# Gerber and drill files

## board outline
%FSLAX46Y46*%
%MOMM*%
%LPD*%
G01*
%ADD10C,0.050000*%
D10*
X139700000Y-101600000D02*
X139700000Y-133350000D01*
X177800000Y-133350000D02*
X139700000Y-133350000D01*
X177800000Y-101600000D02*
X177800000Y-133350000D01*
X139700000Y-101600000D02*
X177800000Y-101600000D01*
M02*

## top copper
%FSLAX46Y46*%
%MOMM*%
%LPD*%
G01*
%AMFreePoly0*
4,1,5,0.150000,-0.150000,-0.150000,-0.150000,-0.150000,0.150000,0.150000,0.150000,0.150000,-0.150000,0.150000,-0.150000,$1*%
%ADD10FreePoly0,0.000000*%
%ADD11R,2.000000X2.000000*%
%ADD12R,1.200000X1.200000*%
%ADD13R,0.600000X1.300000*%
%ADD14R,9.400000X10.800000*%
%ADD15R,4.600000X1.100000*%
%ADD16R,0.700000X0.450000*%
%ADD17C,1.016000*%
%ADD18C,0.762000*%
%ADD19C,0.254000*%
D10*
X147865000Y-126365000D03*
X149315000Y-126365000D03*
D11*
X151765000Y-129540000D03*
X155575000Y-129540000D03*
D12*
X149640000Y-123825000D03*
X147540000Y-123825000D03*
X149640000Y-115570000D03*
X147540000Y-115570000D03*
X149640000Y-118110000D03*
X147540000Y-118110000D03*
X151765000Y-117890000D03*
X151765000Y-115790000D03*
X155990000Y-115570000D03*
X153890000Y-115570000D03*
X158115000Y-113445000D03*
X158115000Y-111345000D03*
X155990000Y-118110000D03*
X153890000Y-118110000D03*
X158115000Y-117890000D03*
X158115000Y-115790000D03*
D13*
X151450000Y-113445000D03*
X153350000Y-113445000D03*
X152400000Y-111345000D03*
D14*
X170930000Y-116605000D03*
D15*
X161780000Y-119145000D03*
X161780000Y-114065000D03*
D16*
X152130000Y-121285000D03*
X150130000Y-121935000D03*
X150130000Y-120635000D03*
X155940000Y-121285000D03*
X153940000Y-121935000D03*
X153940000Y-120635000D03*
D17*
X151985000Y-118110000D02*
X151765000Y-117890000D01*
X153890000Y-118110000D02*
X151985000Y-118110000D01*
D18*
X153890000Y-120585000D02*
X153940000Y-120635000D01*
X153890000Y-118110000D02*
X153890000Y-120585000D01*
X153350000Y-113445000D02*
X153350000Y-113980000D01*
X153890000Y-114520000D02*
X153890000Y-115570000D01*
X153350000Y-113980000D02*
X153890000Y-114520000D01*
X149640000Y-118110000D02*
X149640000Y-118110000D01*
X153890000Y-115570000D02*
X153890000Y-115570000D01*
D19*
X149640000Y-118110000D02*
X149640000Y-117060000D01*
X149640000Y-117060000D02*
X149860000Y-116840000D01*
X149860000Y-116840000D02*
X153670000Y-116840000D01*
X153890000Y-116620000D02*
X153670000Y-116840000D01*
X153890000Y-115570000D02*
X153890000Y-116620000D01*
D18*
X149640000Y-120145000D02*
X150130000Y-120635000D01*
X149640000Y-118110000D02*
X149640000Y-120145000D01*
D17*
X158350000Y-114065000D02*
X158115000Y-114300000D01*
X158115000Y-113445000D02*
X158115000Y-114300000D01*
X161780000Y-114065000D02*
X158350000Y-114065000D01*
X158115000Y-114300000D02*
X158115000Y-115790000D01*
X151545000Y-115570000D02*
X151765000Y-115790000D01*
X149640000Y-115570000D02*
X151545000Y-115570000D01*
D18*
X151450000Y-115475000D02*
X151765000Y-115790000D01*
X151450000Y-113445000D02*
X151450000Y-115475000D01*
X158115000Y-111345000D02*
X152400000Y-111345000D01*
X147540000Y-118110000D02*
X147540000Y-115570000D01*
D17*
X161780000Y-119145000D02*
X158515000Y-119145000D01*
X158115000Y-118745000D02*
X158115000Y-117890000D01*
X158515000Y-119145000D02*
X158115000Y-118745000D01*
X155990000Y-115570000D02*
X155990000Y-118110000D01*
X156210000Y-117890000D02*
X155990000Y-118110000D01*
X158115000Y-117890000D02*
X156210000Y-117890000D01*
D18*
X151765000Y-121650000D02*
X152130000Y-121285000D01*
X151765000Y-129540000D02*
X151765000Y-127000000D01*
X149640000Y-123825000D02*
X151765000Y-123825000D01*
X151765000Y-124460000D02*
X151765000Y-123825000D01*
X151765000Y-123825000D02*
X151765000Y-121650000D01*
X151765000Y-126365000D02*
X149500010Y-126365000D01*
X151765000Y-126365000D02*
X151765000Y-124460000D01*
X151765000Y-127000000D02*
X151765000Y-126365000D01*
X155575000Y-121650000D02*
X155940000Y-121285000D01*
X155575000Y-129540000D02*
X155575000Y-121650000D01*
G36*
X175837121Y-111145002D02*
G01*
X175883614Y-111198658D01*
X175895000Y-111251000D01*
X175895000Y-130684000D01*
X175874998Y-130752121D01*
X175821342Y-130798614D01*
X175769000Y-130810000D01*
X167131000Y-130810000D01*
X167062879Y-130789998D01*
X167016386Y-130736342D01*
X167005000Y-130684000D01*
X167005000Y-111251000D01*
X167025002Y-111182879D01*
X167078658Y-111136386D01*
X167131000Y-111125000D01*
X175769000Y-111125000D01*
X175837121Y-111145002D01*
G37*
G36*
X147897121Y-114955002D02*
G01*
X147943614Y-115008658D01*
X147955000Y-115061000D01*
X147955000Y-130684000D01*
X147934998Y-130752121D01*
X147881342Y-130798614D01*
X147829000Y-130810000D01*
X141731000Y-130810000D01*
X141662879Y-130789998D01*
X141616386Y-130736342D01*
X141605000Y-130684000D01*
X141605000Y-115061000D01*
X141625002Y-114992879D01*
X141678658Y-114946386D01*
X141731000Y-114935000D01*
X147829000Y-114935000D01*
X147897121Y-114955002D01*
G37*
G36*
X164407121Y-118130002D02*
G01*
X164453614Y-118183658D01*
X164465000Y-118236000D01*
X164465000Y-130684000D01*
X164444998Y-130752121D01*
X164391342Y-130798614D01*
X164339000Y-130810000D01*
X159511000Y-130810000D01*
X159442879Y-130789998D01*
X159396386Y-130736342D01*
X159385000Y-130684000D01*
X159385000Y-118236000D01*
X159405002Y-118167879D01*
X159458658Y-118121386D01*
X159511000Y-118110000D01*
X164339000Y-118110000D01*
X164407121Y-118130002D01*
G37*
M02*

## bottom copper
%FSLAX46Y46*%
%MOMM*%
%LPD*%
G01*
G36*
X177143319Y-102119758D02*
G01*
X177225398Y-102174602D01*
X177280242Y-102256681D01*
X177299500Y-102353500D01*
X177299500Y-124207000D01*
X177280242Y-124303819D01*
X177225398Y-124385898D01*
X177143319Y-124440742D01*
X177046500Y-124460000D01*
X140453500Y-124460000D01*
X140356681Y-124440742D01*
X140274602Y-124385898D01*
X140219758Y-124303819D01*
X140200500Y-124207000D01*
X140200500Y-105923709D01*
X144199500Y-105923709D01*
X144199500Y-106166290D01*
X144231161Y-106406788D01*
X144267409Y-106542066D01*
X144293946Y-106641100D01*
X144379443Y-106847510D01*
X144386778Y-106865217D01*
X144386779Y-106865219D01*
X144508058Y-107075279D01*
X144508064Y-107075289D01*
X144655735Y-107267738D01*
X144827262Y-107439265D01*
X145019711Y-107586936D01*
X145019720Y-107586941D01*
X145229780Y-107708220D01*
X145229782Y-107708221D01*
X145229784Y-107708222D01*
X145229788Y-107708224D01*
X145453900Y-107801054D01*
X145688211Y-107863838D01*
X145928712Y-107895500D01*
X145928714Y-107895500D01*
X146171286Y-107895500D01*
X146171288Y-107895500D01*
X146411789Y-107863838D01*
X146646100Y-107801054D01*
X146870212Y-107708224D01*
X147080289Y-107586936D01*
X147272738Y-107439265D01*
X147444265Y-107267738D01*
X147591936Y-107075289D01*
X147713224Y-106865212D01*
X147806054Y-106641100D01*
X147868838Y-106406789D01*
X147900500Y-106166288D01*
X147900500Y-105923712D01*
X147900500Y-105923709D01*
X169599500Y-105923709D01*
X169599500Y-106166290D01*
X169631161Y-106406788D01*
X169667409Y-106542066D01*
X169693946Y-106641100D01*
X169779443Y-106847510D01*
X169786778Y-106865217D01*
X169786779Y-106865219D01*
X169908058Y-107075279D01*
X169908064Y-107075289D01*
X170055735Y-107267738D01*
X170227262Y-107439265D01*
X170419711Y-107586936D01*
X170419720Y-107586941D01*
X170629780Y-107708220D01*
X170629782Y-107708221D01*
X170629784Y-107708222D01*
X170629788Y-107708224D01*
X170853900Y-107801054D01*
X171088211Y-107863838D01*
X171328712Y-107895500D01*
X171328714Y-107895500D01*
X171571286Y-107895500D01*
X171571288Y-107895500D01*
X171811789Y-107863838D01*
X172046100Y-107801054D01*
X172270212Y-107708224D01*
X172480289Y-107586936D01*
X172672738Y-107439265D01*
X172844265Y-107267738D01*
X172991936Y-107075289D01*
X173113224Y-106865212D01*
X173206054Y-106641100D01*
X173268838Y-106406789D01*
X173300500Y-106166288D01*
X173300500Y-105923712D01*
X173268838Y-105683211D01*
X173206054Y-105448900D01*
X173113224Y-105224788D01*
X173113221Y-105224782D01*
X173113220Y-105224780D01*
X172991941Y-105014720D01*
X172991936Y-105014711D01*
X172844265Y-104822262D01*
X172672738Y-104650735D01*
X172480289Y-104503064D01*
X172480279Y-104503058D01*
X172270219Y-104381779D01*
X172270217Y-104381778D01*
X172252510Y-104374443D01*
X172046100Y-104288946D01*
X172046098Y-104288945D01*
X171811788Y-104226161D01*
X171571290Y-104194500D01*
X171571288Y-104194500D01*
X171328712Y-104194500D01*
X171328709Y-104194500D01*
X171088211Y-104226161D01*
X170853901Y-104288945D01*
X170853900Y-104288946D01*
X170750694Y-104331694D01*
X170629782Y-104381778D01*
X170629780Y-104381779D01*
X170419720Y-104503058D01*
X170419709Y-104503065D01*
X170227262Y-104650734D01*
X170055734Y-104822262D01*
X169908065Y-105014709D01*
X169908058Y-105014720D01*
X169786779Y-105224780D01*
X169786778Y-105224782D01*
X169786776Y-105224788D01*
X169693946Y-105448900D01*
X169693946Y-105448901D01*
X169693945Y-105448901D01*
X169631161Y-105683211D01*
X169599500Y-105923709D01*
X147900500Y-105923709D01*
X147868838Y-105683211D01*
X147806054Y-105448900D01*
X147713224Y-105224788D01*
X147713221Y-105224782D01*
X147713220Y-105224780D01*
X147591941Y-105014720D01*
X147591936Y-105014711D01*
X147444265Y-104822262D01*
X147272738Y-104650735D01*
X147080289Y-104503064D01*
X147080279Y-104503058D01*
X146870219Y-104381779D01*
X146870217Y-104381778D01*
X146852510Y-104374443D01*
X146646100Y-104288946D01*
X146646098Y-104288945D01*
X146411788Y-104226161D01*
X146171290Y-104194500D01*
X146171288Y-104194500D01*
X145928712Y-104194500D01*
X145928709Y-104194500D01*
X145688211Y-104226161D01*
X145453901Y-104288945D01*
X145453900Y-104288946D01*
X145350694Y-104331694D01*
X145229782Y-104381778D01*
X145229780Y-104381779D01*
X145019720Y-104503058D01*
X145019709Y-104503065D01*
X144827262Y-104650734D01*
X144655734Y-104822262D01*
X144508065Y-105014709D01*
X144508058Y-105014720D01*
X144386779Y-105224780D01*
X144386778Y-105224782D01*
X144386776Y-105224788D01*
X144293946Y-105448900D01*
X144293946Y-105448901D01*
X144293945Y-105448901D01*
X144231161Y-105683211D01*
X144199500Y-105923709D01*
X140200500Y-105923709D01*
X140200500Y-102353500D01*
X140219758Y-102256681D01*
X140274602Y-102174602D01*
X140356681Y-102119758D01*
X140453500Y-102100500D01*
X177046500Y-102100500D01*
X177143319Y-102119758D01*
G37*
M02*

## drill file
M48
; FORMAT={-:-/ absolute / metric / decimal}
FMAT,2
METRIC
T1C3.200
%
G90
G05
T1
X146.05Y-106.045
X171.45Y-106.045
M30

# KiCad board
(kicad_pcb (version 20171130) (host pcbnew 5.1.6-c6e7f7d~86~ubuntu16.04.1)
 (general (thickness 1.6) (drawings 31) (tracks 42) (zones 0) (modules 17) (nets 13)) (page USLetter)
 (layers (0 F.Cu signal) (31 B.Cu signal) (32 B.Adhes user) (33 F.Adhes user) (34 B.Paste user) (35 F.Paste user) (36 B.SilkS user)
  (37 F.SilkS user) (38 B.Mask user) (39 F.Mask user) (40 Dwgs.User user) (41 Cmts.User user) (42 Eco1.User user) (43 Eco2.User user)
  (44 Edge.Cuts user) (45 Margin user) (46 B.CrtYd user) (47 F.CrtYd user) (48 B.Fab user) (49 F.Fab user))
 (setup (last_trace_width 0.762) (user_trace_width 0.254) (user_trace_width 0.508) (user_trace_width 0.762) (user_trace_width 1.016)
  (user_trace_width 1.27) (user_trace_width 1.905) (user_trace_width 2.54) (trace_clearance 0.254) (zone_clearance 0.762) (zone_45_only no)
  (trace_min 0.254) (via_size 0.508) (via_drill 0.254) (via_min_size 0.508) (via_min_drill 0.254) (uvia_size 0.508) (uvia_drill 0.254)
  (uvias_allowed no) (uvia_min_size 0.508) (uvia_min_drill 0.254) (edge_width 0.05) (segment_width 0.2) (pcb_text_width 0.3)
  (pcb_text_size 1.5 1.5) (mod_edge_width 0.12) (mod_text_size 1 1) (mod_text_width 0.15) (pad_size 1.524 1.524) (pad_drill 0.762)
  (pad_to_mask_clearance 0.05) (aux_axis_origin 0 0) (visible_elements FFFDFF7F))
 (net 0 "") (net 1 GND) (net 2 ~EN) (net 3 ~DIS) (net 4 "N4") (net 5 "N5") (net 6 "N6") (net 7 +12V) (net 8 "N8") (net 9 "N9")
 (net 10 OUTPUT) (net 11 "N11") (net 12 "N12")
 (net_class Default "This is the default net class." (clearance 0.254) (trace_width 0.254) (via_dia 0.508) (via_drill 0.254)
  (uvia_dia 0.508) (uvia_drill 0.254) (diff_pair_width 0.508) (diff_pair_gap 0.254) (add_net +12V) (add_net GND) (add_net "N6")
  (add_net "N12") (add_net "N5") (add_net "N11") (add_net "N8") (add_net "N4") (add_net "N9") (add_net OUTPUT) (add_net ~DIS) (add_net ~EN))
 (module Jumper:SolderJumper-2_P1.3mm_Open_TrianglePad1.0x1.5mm (layer F.Cu) (at 148.59 126.365)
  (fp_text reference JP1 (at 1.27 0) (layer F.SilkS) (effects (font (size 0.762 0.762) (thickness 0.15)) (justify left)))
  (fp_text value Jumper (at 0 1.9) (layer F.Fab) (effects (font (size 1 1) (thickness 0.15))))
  (pad 1 smd custom (at -0.725 0) (size 0.3 0.3) (layers F.Cu F.Mask) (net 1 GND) (zone_connect 2)
   (options (clearance outline) (anchor rect)) (primitives))
  (pad 2 smd custom (at 0.725 0) (size 0.3 0.3) (layers F.Cu F.Mask) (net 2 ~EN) (zone_connect 2)
   (options (clearance outline) (anchor rect)) (primitives)))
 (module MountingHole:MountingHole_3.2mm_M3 (layer F.Cu) (at 171.45 106.045)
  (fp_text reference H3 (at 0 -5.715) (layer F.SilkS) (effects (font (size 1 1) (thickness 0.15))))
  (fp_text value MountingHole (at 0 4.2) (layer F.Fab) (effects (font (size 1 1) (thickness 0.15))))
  (pad 1 np_thru_hole circle (at 0 0) (size 3.2 3.2) (drill 3.2) (layers *.Cu *.Mask)))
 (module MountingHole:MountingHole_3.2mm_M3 (layer F.Cu) (at 146.05 106.045)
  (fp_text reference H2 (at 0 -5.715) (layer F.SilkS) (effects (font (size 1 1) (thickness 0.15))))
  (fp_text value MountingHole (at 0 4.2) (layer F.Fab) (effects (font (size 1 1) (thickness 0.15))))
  (pad 1 np_thru_hole circle (at 0 0) (size 3.2 3.2) (drill 3.2) (layers *.Cu *.Mask)))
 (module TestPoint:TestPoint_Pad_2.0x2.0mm (layer F.Cu) (at 151.765 129.54 180)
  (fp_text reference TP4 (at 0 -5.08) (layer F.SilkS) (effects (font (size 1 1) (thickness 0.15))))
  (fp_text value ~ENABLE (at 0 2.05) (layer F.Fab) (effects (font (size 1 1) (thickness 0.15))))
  (pad 1 smd rect (at 0 0 180) (size 2 2) (layers F.Cu F.Mask) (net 2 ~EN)))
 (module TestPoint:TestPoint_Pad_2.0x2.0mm (layer F.Cu) (at 155.575 129.54 180)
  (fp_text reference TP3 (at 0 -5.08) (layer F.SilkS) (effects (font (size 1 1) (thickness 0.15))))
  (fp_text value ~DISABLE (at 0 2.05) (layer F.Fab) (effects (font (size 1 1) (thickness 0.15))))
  (pad 1 smd rect (at 0 0 180) (size 2 2) (layers F.Cu F.Mask) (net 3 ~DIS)))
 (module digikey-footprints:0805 (layer F.Cu) (at 148.59 123.825 180)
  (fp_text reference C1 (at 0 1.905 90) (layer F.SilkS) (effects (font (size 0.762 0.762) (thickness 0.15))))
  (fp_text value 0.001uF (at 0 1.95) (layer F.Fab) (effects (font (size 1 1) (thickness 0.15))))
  (pad 1 smd rect (at -1.05 0 180) (size 1.2 1.2) (layers F.Cu F.Paste F.Mask) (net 2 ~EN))
  (pad 2 smd rect (at 1.05 0 180) (size 1.2 1.2) (layers F.Cu F.Paste F.Mask) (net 1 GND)))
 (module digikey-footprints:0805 (layer F.Cu) (at 148.59 115.57 180)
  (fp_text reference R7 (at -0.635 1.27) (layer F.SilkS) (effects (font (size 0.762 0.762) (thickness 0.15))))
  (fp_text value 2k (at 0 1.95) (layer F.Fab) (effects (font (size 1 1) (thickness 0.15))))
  (pad 1 smd rect (at -1.05 0 180) (size 1.2 1.2) (layers F.Cu F.Paste F.Mask) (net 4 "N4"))
  (pad 2 smd rect (at 1.05 0 180) (size 1.2 1.2) (layers F.Cu F.Paste F.Mask) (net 1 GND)))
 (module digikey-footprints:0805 (layer F.Cu) (at 148.59 118.11 180)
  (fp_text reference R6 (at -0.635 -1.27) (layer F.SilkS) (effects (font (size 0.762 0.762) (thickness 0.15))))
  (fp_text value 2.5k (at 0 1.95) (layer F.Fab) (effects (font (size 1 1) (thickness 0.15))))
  (pad 1 smd rect (at -1.05 0 180) (size 1.2 1.2) (layers F.Cu F.Paste F.Mask) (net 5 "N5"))
  (pad 2 smd rect (at 1.05 0 180) (size 1.2 1.2) (layers F.Cu F.Paste F.Mask) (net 1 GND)))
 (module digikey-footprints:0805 (layer F.Cu) (at 151.765 116.84 90)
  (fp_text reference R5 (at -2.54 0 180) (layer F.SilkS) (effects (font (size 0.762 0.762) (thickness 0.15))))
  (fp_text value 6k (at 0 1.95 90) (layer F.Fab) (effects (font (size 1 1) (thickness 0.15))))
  (pad 1 smd rect (at -1.05 0 90) (size 1.2 1.2) (layers F.Cu F.Paste F.Mask) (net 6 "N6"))
  (pad 2 smd rect (at 1.05 0 90) (size 1.2 1.2) (layers F.Cu F.Paste F.Mask) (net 4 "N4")))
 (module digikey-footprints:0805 (layer F.Cu) (at 154.94 115.57 180)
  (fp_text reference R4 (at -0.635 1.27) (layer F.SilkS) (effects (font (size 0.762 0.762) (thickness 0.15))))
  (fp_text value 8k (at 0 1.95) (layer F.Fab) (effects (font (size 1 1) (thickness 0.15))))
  (pad 1 smd rect (at -1.05 0 180) (size 1.2 1.2) (layers F.Cu F.Paste F.Mask) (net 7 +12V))
  (pad 2 smd rect (at 1.05 0 180) (size 1.2 1.2) (layers F.Cu F.Paste F.Mask) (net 5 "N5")))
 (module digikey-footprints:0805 (layer F.Cu) (at 158.115 112.395 90)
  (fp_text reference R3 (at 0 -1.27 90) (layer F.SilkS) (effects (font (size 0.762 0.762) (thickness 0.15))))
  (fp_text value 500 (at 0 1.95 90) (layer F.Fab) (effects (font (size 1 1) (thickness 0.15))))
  (pad 1 smd rect (at -1.05 0 90) (size 1.2 1.2) (layers F.Cu F.Paste F.Mask) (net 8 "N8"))
  (pad 2 smd rect (at 1.05 0 90) (size 1.2 1.2) (layers F.Cu F.Paste F.Mask) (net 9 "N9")))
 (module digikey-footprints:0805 (layer F.Cu) (at 154.94 118.11 180)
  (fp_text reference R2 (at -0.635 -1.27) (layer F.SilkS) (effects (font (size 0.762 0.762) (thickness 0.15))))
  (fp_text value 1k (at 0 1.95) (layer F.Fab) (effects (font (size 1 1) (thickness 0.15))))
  (pad 1 smd rect (at -1.05 0 180) (size 1.2 1.2) (layers F.Cu F.Paste F.Mask) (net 7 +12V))
  (pad 2 smd rect (at 1.05 0 180) (size 1.2 1.2) (layers F.Cu F.Paste F.Mask) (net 6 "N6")))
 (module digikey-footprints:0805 (layer F.Cu) (at 158.115 116.84 90)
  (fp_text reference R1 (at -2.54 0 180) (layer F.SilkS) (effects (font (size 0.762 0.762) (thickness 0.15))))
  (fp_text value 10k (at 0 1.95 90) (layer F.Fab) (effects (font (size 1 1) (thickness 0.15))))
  (pad 1 smd rect (at -1.05 0 90) (size 1.2 1.2) (layers F.Cu F.Paste F.Mask) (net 7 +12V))
  (pad 2 smd rect (at 1.05 0 90) (size 1.2 1.2) (layers F.Cu F.Paste F.Mask) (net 8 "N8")))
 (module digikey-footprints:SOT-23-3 (layer F.Cu) (at 152.4 112.395 90)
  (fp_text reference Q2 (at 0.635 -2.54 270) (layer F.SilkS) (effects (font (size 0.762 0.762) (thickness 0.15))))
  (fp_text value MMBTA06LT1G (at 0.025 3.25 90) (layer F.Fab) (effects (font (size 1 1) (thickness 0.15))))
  (pad 1 smd rect (at -1.05 -0.95 90) (size 1.3 0.6) (layers F.Cu F.Paste F.Mask) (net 4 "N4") (solder_mask_margin 0.07))
  (pad 2 smd rect (at -1.05 0.95 90) (size 1.3 0.6) (layers F.Cu F.Paste F.Mask) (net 5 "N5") (solder_mask_margin 0.07))
  (pad 3 smd rect (at 1.05 0 90) (size 1.3 0.6) (layers F.Cu F.Paste F.Mask) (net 9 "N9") (solder_mask_margin 0.07)))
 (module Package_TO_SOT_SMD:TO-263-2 (layer F.Cu) (at 167.555 116.605)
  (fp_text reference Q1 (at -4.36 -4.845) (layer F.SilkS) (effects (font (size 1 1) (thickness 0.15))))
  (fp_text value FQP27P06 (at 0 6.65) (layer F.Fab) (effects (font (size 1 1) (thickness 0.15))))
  (pad "" smd rect (at 0.95 2.775) (size 4.55 5.25) (layers F.Paste))
  (pad "" smd rect (at 5.8 -2.775) (size 4.55 5.25) (layers F.Paste))
  (pad "" smd rect (at 0.95 -2.775) (size 4.55 5.25) (layers F.Paste))
  (pad "" smd rect (at 5.8 2.775) (size 4.55 5.25) (layers F.Paste))
  (pad 2 smd rect (at 3.375 0) (size 9.4 10.8) (layers F.Cu F.Mask) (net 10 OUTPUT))
  (pad 3 smd rect (at -5.775 2.54) (size 4.6 1.1) (layers F.Cu F.Paste F.Mask) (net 7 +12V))
  (pad 1 smd rect (at -5.775 -2.54) (size 4.6 1.1) (layers F.Cu F.Paste F.Mask) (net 8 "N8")))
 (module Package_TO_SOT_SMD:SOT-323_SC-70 (layer F.Cu) (at 151.13 121.285)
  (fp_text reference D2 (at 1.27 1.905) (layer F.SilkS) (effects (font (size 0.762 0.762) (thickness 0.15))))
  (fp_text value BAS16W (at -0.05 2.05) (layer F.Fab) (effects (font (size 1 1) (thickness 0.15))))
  (pad 3 smd rect (at 1 0 270) (size 0.45 0.7) (layers F.Cu F.Paste F.Mask) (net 2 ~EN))
  (pad 2 smd rect (at -1 0.65 270) (size 0.45 0.7) (layers F.Cu F.Paste F.Mask) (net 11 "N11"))
  (pad 1 smd rect (at -1 -0.65 270) (size 0.45 0.7) (layers F.Cu F.Paste F.Mask) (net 5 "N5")))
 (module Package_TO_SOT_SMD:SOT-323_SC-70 (layer F.Cu) (at 154.94 121.285)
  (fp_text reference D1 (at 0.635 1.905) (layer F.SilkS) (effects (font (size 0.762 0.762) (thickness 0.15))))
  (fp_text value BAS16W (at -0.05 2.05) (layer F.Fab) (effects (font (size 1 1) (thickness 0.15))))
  (pad 3 smd rect (at 1 0 270) (size 0.45 0.7) (layers F.Cu F.Paste F.Mask) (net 3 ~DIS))
  (pad 2 smd rect (at -1 0.65 270) (size 0.45 0.7) (layers F.Cu F.Paste F.Mask) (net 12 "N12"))
  (pad 1 smd rect (at -1 -0.65 270) (size 0.45 0.7) (layers F.Cu F.Paste F.Mask) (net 6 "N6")))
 (gr_line (start 139.7 101.6) (end 139.7 133.35) (layer Edge.Cuts) (width 0.05))
 (gr_line (start 177.8 133.35) (end 139.7 133.35) (layer Edge.Cuts) (width 0.05))
 (gr_line (start 177.8 101.6) (end 177.8 133.35) (layer Edge.Cuts) (width 0.05))
 (gr_line (start 139.7 101.6) (end 177.8 101.6) (layer Edge.Cuts) (width 0.05))
 (segment (start 151.985 118.11) (end 151.765 117.89) (width 1.016) (layer F.Cu) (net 6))
 (segment (start 153.89 118.11) (end 151.985 118.11) (width 1.016) (layer F.Cu) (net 6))
 (segment (start 153.89 120.585) (end 153.94 120.635) (width 0.762) (layer F.Cu) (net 6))
 (segment (start 153.89 118.11) (end 153.89 120.585) (width 0.762) (layer F.Cu) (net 6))
 (segment (start 153.35 113.445) (end 153.35 113.98) (width 0.762) (layer F.Cu) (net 5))
 (segment (start 153.89 114.52) (end 153.89 115.57) (width 0.762) (layer F.Cu) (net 5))
 (segment (start 153.35 113.98) (end 153.89 114.52) (width 0.762) (layer F.Cu) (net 5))
 (segment (start 149.64 118.11) (end 149.64 118.11) (width 0.762) (layer F.Cu) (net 5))
 (segment (start 153.89 115.57) (end 153.89 115.57) (width 0.762) (layer F.Cu) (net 5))
 (segment (start 149.64 118.11) (end 149.64 117.06) (width 0.254) (layer F.Cu) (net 5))
 (segment (start 149.64 117.06) (end 149.86 116.84) (width 0.254) (layer F.Cu) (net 5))
 (segment (start 149.86 116.84) (end 153.67 116.84) (width 0.254) (layer F.Cu) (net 5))
 (segment (start 153.89 116.62) (end 153.67 116.84) (width 0.254) (layer F.Cu) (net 5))
 (segment (start 153.89 115.57) (end 153.89 116.62) (width 0.254) (layer F.Cu) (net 5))
 (segment (start 149.64 120.145) (end 150.13 120.635) (width 0.762) (layer F.Cu) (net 5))
 (segment (start 149.64 118.11) (end 149.64 120.145) (width 0.762) (layer F.Cu) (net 5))
 (segment (start 158.35 114.065) (end 158.115 114.3) (width 1.016) (layer F.Cu) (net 8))
 (segment (start 158.115 113.445) (end 158.115 114.3) (width 1.016) (layer F.Cu) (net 8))
 (segment (start 161.78 114.065) (end 158.35 114.065) (width 1.016) (layer F.Cu) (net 8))
 (segment (start 158.115 114.3) (end 158.115 115.79) (width 1.016) (layer F.Cu) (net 8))
 (segment (start 151.545 115.57) (end 151.765 115.79) (width 1.016) (layer F.Cu) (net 4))
 (segment (start 149.64 115.57) (end 151.545 115.57) (width 1.016) (layer F.Cu) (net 4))
 (segment (start 151.45 115.475) (end 151.765 115.79) (width 0.762) (layer F.Cu) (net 4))
 (segment (start 151.45 113.445) (end 151.45 115.475) (width 0.762) (layer F.Cu) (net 4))
 (segment (start 158.115 111.345) (end 152.4 111.345) (width 0.762) (layer F.Cu) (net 9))
 (segment (start 147.54 118.11) (end 147.54 115.57) (width 0.762) (layer F.Cu) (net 1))
 (segment (start 161.78 119.145) (end 158.515 119.145) (width 1.016) (layer F.Cu) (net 7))
 (segment (start 158.115 118.745) (end 158.115 117.89) (width 1.016) (layer F.Cu) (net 7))
 (segment (start 158.515 119.145) (end 158.115 118.745) (width 1.016) (layer F.Cu) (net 7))
 (segment (start 155.99 115.57) (end 155.99 118.11) (width 1.016) (layer F.Cu) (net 7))
 (segment (start 156.21 117.89) (end 155.99 118.11) (width 1.016) (layer F.Cu) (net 7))
 (segment (start 158.115 117.89) (end 156.21 117.89) (width 1.016) (layer F.Cu) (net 7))
 (segment (start 151.765 121.65) (end 152.13 121.285) (width 0.762) (layer F.Cu) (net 2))
 (segment (start 151.765 129.54) (end 151.765 127) (width 0.762) (layer F.Cu) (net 2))
 (segment (start 149.64 123.825) (end 151.765 123.825) (width 0.762) (layer F.Cu) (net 2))
 (segment (start 151.765 124.46) (end 151.765 123.825) (width 0.762) (layer F.Cu) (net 2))
 (segment (start 151.765 123.825) (end 151.765 121.65) (width 0.762) (layer F.Cu) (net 2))
 (segment (start 151.765 126.365) (end 149.50001 126.365) (width 0.762) (layer F.Cu) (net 2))
 (segment (start 151.765 126.365) (end 151.765 124.46) (width 0.762) (layer F.Cu) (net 2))
 (segment (start 151.765 127) (end 151.765 126.365) (width 0.762) (layer F.Cu) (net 2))
 (segment (start 155.575 121.65) (end 155.94 121.285) (width 0.762) (layer F.Cu) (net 3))
 (segment (start 155.575 129.54) (end 155.575 121.65) (width 0.762) (layer F.Cu) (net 3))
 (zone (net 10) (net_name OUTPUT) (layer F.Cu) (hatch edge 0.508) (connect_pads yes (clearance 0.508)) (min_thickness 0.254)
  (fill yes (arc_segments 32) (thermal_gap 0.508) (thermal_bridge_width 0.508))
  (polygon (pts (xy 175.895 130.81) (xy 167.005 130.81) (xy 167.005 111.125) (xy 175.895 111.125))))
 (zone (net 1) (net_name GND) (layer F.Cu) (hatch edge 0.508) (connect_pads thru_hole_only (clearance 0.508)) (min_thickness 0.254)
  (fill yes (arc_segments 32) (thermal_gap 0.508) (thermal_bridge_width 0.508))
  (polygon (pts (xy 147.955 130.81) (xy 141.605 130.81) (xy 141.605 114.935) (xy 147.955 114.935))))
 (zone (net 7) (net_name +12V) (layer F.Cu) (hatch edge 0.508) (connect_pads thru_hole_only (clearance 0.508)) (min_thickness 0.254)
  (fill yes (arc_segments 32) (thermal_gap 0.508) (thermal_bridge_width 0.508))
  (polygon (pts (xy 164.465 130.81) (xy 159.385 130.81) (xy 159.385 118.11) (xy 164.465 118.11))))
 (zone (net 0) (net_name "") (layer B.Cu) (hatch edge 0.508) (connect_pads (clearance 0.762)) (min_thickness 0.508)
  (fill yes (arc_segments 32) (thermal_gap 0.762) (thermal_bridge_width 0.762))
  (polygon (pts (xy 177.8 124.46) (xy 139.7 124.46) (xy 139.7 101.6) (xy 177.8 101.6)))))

